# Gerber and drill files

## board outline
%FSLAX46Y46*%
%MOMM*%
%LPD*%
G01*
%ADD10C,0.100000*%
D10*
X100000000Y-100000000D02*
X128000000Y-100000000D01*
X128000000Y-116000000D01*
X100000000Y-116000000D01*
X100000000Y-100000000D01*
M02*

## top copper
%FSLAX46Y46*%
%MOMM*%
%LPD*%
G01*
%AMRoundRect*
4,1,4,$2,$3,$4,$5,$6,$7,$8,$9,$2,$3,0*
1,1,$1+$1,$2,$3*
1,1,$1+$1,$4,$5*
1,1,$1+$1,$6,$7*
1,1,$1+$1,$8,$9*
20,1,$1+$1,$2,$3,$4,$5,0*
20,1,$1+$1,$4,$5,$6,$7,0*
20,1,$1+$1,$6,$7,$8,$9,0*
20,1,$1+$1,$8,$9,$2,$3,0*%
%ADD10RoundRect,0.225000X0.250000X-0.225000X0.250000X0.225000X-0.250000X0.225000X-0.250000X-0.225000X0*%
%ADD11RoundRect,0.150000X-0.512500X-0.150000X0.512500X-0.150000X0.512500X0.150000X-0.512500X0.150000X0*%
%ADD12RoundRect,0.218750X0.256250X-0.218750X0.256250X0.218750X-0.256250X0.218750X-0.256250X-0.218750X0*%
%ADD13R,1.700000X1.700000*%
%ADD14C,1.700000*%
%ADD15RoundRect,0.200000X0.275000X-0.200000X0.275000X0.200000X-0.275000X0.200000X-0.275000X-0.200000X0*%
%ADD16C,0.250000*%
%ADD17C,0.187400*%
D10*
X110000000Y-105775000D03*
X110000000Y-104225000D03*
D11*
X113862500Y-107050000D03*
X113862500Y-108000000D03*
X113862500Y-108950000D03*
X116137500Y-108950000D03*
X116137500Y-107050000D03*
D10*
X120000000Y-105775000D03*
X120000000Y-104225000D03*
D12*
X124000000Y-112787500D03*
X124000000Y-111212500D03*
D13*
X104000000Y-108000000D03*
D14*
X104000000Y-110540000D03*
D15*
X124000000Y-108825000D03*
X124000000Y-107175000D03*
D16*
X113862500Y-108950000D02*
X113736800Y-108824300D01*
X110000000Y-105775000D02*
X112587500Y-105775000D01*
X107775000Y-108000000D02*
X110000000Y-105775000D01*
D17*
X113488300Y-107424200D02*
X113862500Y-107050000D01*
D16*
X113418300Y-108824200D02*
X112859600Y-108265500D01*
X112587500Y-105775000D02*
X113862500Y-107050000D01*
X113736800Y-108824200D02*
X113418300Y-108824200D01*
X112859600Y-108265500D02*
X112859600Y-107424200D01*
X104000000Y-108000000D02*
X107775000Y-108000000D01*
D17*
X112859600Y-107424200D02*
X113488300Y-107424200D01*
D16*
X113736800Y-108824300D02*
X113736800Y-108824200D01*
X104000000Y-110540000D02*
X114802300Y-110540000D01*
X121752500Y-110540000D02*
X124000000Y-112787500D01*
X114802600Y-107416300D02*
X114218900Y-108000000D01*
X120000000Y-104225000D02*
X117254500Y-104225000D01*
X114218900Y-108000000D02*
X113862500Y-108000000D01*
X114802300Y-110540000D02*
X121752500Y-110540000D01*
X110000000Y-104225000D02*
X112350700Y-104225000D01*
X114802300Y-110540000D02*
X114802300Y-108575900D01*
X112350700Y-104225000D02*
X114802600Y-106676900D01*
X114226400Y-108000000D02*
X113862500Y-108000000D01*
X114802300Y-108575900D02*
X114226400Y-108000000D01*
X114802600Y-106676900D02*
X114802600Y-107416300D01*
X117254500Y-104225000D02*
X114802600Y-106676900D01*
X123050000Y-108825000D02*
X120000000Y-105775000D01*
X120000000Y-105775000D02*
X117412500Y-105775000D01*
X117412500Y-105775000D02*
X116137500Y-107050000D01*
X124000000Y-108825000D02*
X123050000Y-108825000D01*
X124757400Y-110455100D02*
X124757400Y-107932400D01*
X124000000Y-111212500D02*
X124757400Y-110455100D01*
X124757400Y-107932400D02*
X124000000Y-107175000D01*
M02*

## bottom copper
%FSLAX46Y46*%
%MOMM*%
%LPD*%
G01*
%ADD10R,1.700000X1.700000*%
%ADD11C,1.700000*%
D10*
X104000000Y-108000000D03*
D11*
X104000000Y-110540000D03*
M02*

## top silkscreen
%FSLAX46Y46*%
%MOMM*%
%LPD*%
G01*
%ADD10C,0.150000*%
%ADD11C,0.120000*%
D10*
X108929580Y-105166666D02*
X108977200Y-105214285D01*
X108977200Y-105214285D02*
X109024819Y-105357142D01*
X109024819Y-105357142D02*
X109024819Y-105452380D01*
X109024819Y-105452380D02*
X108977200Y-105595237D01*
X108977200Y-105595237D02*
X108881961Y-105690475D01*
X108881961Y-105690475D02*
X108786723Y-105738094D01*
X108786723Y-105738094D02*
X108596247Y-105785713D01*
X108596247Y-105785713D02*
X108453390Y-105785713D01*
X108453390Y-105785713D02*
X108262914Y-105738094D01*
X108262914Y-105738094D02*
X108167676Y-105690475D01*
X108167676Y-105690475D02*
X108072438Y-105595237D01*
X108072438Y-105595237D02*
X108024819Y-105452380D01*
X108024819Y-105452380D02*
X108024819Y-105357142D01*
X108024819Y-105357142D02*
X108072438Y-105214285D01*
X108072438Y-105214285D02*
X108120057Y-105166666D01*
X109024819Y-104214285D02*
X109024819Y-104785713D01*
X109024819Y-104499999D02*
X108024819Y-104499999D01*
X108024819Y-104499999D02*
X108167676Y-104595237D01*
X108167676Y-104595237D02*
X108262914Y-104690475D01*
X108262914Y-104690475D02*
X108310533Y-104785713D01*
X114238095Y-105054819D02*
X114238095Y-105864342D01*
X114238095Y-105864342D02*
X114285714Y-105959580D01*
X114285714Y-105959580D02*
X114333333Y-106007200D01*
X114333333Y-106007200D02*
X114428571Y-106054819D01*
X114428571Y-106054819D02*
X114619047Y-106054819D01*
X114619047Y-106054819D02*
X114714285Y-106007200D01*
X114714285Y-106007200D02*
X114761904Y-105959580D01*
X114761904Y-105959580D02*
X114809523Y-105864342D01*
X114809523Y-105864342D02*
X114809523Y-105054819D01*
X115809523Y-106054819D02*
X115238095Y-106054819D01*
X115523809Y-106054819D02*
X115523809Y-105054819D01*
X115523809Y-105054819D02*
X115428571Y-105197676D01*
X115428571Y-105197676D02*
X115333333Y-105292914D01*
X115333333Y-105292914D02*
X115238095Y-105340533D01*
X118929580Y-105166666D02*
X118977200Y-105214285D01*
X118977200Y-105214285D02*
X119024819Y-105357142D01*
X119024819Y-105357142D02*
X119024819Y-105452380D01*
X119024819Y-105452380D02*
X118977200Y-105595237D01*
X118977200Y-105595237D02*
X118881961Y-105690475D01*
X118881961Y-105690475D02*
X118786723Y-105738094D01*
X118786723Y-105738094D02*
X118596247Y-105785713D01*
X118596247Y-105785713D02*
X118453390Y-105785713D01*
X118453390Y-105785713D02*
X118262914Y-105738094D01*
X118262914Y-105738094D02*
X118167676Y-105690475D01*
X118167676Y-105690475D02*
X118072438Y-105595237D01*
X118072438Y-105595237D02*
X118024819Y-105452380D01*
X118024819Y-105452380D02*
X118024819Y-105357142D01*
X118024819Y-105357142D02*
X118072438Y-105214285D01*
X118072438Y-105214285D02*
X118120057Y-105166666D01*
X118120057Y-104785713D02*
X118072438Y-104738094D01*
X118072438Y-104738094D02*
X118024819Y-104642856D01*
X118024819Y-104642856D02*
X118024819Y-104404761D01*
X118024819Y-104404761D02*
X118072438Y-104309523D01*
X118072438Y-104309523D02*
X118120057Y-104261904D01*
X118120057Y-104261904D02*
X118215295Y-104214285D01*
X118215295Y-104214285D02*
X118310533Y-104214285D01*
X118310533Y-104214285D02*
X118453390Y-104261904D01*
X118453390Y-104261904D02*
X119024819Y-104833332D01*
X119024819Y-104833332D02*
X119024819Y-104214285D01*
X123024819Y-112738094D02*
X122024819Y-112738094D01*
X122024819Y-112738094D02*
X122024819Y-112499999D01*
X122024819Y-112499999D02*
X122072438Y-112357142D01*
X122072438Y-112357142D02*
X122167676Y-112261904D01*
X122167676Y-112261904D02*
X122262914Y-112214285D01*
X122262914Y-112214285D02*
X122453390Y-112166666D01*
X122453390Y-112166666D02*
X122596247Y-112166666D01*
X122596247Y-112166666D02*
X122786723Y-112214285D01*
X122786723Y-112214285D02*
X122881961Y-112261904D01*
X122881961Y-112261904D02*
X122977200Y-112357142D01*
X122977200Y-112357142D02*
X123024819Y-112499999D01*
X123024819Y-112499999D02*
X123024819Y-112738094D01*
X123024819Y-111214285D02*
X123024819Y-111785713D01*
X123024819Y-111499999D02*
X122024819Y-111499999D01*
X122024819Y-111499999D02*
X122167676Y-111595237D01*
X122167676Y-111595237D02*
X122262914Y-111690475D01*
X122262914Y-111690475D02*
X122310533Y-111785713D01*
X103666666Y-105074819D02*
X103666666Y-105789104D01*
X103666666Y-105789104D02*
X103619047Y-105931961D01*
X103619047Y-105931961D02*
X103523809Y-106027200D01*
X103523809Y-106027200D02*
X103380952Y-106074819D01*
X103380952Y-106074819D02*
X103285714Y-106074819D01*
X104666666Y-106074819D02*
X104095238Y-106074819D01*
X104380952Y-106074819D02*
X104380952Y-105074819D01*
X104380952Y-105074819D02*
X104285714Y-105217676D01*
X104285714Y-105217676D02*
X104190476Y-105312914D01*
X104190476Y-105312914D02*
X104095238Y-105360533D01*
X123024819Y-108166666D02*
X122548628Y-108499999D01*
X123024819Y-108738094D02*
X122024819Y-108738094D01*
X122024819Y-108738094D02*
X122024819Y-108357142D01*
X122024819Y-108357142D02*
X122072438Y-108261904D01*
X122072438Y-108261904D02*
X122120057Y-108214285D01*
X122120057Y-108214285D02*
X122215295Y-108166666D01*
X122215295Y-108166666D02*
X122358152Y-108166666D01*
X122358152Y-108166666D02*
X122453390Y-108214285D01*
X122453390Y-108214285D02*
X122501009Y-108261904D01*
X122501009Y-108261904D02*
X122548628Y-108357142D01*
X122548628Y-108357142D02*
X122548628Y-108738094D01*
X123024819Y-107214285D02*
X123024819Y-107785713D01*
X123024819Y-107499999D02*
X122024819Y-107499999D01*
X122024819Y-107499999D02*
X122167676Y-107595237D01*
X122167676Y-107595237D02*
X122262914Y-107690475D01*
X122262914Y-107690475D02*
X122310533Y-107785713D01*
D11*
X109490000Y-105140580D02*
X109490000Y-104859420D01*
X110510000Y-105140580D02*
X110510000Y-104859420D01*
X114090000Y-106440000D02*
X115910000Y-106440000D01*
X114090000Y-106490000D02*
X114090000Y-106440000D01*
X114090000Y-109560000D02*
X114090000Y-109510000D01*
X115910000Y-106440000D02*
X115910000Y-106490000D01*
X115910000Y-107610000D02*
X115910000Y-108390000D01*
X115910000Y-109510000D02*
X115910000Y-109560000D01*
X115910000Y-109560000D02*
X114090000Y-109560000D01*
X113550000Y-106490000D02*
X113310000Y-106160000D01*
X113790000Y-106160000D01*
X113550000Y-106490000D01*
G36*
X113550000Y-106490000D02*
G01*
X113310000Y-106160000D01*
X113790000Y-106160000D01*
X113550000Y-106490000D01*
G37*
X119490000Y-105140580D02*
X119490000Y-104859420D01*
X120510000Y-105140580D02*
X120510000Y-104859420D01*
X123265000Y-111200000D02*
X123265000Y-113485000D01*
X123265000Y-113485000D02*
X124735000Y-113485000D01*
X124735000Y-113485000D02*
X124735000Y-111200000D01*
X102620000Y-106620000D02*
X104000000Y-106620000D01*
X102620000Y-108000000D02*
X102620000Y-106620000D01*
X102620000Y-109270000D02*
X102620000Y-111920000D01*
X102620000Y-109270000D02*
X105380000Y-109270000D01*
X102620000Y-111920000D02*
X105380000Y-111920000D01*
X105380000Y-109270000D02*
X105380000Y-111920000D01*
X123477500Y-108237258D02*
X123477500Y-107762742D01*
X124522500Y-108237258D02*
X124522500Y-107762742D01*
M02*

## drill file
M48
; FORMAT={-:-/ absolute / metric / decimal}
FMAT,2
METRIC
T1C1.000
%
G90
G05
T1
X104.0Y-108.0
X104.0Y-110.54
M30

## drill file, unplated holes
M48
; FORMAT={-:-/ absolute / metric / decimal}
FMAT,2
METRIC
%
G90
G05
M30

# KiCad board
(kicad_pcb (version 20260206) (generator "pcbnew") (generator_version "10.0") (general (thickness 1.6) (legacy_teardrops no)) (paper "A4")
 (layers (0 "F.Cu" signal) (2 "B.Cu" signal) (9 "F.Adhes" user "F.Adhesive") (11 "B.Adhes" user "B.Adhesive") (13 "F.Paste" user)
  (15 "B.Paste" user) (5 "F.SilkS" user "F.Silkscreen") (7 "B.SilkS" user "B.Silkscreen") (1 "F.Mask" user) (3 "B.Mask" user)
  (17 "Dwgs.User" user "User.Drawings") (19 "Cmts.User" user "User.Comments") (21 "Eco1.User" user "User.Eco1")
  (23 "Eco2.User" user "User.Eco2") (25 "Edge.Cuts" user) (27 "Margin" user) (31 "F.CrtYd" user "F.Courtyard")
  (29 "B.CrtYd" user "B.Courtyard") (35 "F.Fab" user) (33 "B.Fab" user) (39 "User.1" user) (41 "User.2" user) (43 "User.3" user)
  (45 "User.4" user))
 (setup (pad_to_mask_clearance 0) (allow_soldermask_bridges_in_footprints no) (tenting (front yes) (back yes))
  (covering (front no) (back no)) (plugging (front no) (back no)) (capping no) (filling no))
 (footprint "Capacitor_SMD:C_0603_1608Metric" (layer "F.Cu") (at 110 105 90)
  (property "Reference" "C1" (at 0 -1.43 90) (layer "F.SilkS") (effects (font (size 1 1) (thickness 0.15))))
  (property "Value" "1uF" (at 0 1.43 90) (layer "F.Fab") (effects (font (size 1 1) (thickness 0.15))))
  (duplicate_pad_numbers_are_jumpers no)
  (fp_line (start -0.14058 -0.51) (end 0.14058 -0.51) (stroke (width 0.12) (type solid)) (layer "F.SilkS"))
  (fp_line (start -0.14058 0.51) (end 0.14058 0.51) (stroke (width 0.12) (type solid)) (layer "F.SilkS"))
  (pad "1" smd roundrect (at -0.775 0 90) (size 0.9 0.95) (layers "F.Cu" "F.Mask" "F.Paste") (roundrect_rratio 0.25) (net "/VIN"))
  (pad "2" smd roundrect (at 0.775 0 90) (size 0.9 0.95) (layers "F.Cu" "F.Mask" "F.Paste") (roundrect_rratio 0.25) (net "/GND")))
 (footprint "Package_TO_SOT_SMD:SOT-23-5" (layer "F.Cu") (at 115 108)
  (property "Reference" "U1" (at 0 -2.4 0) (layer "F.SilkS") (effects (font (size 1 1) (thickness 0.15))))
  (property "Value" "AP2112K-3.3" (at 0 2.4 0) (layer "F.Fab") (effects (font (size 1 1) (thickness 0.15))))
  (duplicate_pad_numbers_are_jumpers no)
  (fp_line (start -0.91 -1.56) (end 0.91 -1.56) (stroke (width 0.12) (type solid)) (layer "F.SilkS"))
  (fp_line (start -0.91 -1.51) (end -0.91 -1.56) (stroke (width 0.12) (type solid)) (layer "F.SilkS"))
  (fp_line (start -0.91 1.56) (end -0.91 1.51) (stroke (width 0.12) (type solid)) (layer "F.SilkS"))
  (fp_line (start 0.91 -1.56) (end 0.91 -1.51) (stroke (width 0.12) (type solid)) (layer "F.SilkS"))
  (fp_line (start 0.91 -0.39) (end 0.91 0.39) (stroke (width 0.12) (type solid)) (layer "F.SilkS"))
  (fp_line (start 0.91 1.51) (end 0.91 1.56) (stroke (width 0.12) (type solid)) (layer "F.SilkS"))
  (fp_line (start 0.91 1.56) (end -0.91 1.56) (stroke (width 0.12) (type solid)) (layer "F.SilkS"))
  (fp_poly (pts (xy -1.45 -1.51) (xy -1.69 -1.84) (xy -1.21 -1.84)) (stroke (width 0.12) (type solid)) (fill yes) (layer "F.SilkS"))
  (pad "1" smd roundrect (at -1.1375 -0.95) (size 1.325 0.6) (layers "F.Cu" "F.Mask" "F.Paste") (roundrect_rratio 0.25) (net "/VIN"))
  (pad "2" smd roundrect (at -1.1375 0) (size 1.325 0.6) (layers "F.Cu" "F.Mask" "F.Paste") (roundrect_rratio 0.25) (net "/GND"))
  (pad "3" smd roundrect (at -1.1375 0.95) (size 1.325 0.6) (layers "F.Cu" "F.Mask" "F.Paste") (roundrect_rratio 0.25) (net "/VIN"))
  (pad "4" smd roundrect (at 1.1375 0.95) (size 1.325 0.6) (layers "F.Cu" "F.Mask" "F.Paste") (roundrect_rratio 0.25)
   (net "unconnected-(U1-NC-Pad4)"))
  (pad "5" smd roundrect (at 1.1375 -0.95) (size 1.325 0.6) (layers "F.Cu" "F.Mask" "F.Paste") (roundrect_rratio 0.25) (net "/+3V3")))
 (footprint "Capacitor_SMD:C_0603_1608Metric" (layer "F.Cu") (at 120 105 90)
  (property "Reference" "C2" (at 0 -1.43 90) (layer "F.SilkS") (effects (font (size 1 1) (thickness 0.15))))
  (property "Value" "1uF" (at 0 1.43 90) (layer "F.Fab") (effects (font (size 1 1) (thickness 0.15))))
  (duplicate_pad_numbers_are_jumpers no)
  (fp_line (start -0.14058 -0.51) (end 0.14058 -0.51) (stroke (width 0.12) (type solid)) (layer "F.SilkS"))
  (fp_line (start -0.14058 0.51) (end 0.14058 0.51) (stroke (width 0.12) (type solid)) (layer "F.SilkS"))
  (pad "1" smd roundrect (at -0.775 0 90) (size 0.9 0.95) (layers "F.Cu" "F.Mask" "F.Paste") (roundrect_rratio 0.25) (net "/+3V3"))
  (pad "2" smd roundrect (at 0.775 0 90) (size 0.9 0.95) (layers "F.Cu" "F.Mask" "F.Paste") (roundrect_rratio 0.25) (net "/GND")))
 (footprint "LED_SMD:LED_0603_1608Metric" (layer "F.Cu") (at 124 112 90)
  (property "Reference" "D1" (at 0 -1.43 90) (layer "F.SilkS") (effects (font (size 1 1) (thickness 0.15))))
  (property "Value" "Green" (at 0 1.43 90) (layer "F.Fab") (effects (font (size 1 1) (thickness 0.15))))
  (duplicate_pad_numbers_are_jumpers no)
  (fp_line (start 0.8 -0.735) (end -1.485 -0.735) (stroke (width 0.12) (type solid)) (layer "F.SilkS"))
  (fp_line (start -1.485 -0.735) (end -1.485 0.735) (stroke (width 0.12) (type solid)) (layer "F.SilkS"))
  (fp_line (start -1.485 0.735) (end 0.8 0.735) (stroke (width 0.12) (type solid)) (layer "F.SilkS"))
  (pad "1" smd roundrect (at -0.7875 0 90) (size 0.875 0.95) (layers "F.Cu" "F.Mask" "F.Paste") (roundrect_rratio 0.25) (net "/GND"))
  (pad "2" smd roundrect (at 0.7875 0 90) (size 0.875 0.95) (layers "F.Cu" "F.Mask" "F.Paste") (roundrect_rratio 0.25) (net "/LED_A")))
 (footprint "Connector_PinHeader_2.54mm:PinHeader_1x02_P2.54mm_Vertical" (layer "F.Cu") (at 104 108)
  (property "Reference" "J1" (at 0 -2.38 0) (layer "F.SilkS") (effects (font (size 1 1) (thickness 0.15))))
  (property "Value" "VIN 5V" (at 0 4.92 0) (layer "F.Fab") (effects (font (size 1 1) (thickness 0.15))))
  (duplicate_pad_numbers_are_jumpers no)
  (fp_line (start -1.38 -1.38) (end 0 -1.38) (stroke (width 0.12) (type solid)) (layer "F.SilkS"))
  (fp_line (start -1.38 0) (end -1.38 -1.38) (stroke (width 0.12) (type solid)) (layer "F.SilkS"))
  (fp_line (start -1.38 1.27) (end -1.38 3.92) (stroke (width 0.12) (type solid)) (layer "F.SilkS"))
  (fp_line (start -1.38 1.27) (end 1.38 1.27) (stroke (width 0.12) (type solid)) (layer "F.SilkS"))
  (fp_line (start -1.38 3.92) (end 1.38 3.92) (stroke (width 0.12) (type solid)) (layer "F.SilkS"))
  (fp_line (start 1.38 1.27) (end 1.38 3.92) (stroke (width 0.12) (type solid)) (layer "F.SilkS"))
  (pad "1" thru_hole rect (at 0 0) (size 1.7 1.7) (drill 1) (layers "*.Cu" "*.Mask") (remove_unused_layers no) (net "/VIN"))
  (pad "2" thru_hole circle (at 0 2.54) (size 1.7 1.7) (drill 1) (layers "*.Cu" "*.Mask") (remove_unused_layers no) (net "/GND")))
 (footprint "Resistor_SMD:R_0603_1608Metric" (layer "F.Cu") (at 124 108 90)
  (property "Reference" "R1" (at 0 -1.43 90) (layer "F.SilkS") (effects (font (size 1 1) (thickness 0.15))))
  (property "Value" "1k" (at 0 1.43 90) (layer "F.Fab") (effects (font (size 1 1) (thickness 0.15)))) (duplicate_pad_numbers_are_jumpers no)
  (fp_line (start -0.237258 -0.5225) (end 0.237258 -0.5225) (stroke (width 0.12) (type solid)) (layer "F.SilkS"))
  (fp_line (start -0.237258 0.5225) (end 0.237258 0.5225) (stroke (width 0.12) (type solid)) (layer "F.SilkS"))
  (pad "1" smd roundrect (at -0.825 0 90) (size 0.8 0.95) (layers "F.Cu" "F.Mask" "F.Paste") (roundrect_rratio 0.25) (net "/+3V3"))
  (pad "2" smd roundrect (at 0.825 0 90) (size 0.8 0.95) (layers "F.Cu" "F.Mask" "F.Paste") (roundrect_rratio 0.25) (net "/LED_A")))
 (gr_rect (start 100 100) (end 128 116) (stroke (width 0.1) (type default)) (fill no) (layer "Edge.Cuts"))
 (segment (start 113.8625 108.95) (end 113.7368 108.8243) (width 0.25) (layer "F.Cu") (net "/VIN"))
 (segment (start 110 105.775) (end 112.5875 105.775) (width 0.25) (layer "F.Cu") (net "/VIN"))
 (segment (start 107.775 108) (end 110 105.775) (width 0.25) (layer "F.Cu") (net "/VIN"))
 (segment (start 113.4883 107.4242) (end 113.8625 107.05) (width 0.1874) (layer "F.Cu") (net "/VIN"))
 (segment (start 113.4183 108.8242) (end 112.8596 108.2655) (width 0.25) (layer "F.Cu") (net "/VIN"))
 (segment (start 112.5875 105.775) (end 113.8625 107.05) (width 0.25) (layer "F.Cu") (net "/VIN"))
 (segment (start 113.7368 108.8242) (end 113.4183 108.8242) (width 0.25) (layer "F.Cu") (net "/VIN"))
 (segment (start 112.8596 108.2655) (end 112.8596 107.4242) (width 0.25) (layer "F.Cu") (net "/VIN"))
 (segment (start 104 108) (end 107.775 108) (width 0.25) (layer "F.Cu") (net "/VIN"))
 (segment (start 112.8596 107.4242) (end 113.4883 107.4242) (width 0.1874) (layer "F.Cu") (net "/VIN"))
 (segment (start 113.7368 108.8243) (end 113.7368 108.8242) (width 0.25) (layer "F.Cu") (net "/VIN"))
 (segment (start 104 110.54) (end 114.8023 110.54) (width 0.25) (layer "F.Cu") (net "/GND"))
 (segment (start 121.7525 110.54) (end 124 112.7875) (width 0.25) (layer "F.Cu") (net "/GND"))
 (segment (start 114.8026 107.4163) (end 114.2189 108) (width 0.25) (layer "F.Cu") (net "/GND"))
 (segment (start 120 104.225) (end 117.2545 104.225) (width 0.25) (layer "F.Cu") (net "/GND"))
 (segment (start 114.2189 108) (end 113.8625 108) (width 0.25) (layer "F.Cu") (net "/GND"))
 (segment (start 114.8023 110.54) (end 121.7525 110.54) (width 0.25) (layer "F.Cu") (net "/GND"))
 (segment (start 110 104.225) (end 112.3507 104.225) (width 0.25) (layer "F.Cu") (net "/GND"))
 (segment (start 114.8023 110.54) (end 114.8023 108.5759) (width 0.25) (layer "F.Cu") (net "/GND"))
 (segment (start 112.3507 104.225) (end 114.8026 106.6769) (width 0.25) (layer "F.Cu") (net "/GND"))
 (segment (start 114.2264 108) (end 113.8625 108) (width 0.25) (layer "F.Cu") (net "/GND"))
 (segment (start 114.8023 108.5759) (end 114.2264 108) (width 0.25) (layer "F.Cu") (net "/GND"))
 (segment (start 114.8026 106.6769) (end 114.8026 107.4163) (width 0.25) (layer "F.Cu") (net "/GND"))
 (segment (start 117.2545 104.225) (end 114.8026 106.6769) (width 0.25) (layer "F.Cu") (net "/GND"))
 (segment (start 123.05 108.825) (end 120 105.775) (width 0.25) (layer "F.Cu") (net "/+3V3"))
 (segment (start 120 105.775) (end 117.4125 105.775) (width 0.25) (layer "F.Cu") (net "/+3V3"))
 (segment (start 117.4125 105.775) (end 116.1375 107.05) (width 0.25) (layer "F.Cu") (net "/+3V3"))
 (segment (start 124 108.825) (end 123.05 108.825) (width 0.25) (layer "F.Cu") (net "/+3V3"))
 (segment (start 124.7574 110.4551) (end 124.7574 107.9324) (width 0.25) (layer "F.Cu") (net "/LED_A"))
 (segment (start 124 111.2125) (end 124.7574 110.4551) (width 0.25) (layer "F.Cu") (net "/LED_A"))
 (segment (start 124.7574 107.9324) (end 124 107.175) (width 0.25) (layer "F.Cu") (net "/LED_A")))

